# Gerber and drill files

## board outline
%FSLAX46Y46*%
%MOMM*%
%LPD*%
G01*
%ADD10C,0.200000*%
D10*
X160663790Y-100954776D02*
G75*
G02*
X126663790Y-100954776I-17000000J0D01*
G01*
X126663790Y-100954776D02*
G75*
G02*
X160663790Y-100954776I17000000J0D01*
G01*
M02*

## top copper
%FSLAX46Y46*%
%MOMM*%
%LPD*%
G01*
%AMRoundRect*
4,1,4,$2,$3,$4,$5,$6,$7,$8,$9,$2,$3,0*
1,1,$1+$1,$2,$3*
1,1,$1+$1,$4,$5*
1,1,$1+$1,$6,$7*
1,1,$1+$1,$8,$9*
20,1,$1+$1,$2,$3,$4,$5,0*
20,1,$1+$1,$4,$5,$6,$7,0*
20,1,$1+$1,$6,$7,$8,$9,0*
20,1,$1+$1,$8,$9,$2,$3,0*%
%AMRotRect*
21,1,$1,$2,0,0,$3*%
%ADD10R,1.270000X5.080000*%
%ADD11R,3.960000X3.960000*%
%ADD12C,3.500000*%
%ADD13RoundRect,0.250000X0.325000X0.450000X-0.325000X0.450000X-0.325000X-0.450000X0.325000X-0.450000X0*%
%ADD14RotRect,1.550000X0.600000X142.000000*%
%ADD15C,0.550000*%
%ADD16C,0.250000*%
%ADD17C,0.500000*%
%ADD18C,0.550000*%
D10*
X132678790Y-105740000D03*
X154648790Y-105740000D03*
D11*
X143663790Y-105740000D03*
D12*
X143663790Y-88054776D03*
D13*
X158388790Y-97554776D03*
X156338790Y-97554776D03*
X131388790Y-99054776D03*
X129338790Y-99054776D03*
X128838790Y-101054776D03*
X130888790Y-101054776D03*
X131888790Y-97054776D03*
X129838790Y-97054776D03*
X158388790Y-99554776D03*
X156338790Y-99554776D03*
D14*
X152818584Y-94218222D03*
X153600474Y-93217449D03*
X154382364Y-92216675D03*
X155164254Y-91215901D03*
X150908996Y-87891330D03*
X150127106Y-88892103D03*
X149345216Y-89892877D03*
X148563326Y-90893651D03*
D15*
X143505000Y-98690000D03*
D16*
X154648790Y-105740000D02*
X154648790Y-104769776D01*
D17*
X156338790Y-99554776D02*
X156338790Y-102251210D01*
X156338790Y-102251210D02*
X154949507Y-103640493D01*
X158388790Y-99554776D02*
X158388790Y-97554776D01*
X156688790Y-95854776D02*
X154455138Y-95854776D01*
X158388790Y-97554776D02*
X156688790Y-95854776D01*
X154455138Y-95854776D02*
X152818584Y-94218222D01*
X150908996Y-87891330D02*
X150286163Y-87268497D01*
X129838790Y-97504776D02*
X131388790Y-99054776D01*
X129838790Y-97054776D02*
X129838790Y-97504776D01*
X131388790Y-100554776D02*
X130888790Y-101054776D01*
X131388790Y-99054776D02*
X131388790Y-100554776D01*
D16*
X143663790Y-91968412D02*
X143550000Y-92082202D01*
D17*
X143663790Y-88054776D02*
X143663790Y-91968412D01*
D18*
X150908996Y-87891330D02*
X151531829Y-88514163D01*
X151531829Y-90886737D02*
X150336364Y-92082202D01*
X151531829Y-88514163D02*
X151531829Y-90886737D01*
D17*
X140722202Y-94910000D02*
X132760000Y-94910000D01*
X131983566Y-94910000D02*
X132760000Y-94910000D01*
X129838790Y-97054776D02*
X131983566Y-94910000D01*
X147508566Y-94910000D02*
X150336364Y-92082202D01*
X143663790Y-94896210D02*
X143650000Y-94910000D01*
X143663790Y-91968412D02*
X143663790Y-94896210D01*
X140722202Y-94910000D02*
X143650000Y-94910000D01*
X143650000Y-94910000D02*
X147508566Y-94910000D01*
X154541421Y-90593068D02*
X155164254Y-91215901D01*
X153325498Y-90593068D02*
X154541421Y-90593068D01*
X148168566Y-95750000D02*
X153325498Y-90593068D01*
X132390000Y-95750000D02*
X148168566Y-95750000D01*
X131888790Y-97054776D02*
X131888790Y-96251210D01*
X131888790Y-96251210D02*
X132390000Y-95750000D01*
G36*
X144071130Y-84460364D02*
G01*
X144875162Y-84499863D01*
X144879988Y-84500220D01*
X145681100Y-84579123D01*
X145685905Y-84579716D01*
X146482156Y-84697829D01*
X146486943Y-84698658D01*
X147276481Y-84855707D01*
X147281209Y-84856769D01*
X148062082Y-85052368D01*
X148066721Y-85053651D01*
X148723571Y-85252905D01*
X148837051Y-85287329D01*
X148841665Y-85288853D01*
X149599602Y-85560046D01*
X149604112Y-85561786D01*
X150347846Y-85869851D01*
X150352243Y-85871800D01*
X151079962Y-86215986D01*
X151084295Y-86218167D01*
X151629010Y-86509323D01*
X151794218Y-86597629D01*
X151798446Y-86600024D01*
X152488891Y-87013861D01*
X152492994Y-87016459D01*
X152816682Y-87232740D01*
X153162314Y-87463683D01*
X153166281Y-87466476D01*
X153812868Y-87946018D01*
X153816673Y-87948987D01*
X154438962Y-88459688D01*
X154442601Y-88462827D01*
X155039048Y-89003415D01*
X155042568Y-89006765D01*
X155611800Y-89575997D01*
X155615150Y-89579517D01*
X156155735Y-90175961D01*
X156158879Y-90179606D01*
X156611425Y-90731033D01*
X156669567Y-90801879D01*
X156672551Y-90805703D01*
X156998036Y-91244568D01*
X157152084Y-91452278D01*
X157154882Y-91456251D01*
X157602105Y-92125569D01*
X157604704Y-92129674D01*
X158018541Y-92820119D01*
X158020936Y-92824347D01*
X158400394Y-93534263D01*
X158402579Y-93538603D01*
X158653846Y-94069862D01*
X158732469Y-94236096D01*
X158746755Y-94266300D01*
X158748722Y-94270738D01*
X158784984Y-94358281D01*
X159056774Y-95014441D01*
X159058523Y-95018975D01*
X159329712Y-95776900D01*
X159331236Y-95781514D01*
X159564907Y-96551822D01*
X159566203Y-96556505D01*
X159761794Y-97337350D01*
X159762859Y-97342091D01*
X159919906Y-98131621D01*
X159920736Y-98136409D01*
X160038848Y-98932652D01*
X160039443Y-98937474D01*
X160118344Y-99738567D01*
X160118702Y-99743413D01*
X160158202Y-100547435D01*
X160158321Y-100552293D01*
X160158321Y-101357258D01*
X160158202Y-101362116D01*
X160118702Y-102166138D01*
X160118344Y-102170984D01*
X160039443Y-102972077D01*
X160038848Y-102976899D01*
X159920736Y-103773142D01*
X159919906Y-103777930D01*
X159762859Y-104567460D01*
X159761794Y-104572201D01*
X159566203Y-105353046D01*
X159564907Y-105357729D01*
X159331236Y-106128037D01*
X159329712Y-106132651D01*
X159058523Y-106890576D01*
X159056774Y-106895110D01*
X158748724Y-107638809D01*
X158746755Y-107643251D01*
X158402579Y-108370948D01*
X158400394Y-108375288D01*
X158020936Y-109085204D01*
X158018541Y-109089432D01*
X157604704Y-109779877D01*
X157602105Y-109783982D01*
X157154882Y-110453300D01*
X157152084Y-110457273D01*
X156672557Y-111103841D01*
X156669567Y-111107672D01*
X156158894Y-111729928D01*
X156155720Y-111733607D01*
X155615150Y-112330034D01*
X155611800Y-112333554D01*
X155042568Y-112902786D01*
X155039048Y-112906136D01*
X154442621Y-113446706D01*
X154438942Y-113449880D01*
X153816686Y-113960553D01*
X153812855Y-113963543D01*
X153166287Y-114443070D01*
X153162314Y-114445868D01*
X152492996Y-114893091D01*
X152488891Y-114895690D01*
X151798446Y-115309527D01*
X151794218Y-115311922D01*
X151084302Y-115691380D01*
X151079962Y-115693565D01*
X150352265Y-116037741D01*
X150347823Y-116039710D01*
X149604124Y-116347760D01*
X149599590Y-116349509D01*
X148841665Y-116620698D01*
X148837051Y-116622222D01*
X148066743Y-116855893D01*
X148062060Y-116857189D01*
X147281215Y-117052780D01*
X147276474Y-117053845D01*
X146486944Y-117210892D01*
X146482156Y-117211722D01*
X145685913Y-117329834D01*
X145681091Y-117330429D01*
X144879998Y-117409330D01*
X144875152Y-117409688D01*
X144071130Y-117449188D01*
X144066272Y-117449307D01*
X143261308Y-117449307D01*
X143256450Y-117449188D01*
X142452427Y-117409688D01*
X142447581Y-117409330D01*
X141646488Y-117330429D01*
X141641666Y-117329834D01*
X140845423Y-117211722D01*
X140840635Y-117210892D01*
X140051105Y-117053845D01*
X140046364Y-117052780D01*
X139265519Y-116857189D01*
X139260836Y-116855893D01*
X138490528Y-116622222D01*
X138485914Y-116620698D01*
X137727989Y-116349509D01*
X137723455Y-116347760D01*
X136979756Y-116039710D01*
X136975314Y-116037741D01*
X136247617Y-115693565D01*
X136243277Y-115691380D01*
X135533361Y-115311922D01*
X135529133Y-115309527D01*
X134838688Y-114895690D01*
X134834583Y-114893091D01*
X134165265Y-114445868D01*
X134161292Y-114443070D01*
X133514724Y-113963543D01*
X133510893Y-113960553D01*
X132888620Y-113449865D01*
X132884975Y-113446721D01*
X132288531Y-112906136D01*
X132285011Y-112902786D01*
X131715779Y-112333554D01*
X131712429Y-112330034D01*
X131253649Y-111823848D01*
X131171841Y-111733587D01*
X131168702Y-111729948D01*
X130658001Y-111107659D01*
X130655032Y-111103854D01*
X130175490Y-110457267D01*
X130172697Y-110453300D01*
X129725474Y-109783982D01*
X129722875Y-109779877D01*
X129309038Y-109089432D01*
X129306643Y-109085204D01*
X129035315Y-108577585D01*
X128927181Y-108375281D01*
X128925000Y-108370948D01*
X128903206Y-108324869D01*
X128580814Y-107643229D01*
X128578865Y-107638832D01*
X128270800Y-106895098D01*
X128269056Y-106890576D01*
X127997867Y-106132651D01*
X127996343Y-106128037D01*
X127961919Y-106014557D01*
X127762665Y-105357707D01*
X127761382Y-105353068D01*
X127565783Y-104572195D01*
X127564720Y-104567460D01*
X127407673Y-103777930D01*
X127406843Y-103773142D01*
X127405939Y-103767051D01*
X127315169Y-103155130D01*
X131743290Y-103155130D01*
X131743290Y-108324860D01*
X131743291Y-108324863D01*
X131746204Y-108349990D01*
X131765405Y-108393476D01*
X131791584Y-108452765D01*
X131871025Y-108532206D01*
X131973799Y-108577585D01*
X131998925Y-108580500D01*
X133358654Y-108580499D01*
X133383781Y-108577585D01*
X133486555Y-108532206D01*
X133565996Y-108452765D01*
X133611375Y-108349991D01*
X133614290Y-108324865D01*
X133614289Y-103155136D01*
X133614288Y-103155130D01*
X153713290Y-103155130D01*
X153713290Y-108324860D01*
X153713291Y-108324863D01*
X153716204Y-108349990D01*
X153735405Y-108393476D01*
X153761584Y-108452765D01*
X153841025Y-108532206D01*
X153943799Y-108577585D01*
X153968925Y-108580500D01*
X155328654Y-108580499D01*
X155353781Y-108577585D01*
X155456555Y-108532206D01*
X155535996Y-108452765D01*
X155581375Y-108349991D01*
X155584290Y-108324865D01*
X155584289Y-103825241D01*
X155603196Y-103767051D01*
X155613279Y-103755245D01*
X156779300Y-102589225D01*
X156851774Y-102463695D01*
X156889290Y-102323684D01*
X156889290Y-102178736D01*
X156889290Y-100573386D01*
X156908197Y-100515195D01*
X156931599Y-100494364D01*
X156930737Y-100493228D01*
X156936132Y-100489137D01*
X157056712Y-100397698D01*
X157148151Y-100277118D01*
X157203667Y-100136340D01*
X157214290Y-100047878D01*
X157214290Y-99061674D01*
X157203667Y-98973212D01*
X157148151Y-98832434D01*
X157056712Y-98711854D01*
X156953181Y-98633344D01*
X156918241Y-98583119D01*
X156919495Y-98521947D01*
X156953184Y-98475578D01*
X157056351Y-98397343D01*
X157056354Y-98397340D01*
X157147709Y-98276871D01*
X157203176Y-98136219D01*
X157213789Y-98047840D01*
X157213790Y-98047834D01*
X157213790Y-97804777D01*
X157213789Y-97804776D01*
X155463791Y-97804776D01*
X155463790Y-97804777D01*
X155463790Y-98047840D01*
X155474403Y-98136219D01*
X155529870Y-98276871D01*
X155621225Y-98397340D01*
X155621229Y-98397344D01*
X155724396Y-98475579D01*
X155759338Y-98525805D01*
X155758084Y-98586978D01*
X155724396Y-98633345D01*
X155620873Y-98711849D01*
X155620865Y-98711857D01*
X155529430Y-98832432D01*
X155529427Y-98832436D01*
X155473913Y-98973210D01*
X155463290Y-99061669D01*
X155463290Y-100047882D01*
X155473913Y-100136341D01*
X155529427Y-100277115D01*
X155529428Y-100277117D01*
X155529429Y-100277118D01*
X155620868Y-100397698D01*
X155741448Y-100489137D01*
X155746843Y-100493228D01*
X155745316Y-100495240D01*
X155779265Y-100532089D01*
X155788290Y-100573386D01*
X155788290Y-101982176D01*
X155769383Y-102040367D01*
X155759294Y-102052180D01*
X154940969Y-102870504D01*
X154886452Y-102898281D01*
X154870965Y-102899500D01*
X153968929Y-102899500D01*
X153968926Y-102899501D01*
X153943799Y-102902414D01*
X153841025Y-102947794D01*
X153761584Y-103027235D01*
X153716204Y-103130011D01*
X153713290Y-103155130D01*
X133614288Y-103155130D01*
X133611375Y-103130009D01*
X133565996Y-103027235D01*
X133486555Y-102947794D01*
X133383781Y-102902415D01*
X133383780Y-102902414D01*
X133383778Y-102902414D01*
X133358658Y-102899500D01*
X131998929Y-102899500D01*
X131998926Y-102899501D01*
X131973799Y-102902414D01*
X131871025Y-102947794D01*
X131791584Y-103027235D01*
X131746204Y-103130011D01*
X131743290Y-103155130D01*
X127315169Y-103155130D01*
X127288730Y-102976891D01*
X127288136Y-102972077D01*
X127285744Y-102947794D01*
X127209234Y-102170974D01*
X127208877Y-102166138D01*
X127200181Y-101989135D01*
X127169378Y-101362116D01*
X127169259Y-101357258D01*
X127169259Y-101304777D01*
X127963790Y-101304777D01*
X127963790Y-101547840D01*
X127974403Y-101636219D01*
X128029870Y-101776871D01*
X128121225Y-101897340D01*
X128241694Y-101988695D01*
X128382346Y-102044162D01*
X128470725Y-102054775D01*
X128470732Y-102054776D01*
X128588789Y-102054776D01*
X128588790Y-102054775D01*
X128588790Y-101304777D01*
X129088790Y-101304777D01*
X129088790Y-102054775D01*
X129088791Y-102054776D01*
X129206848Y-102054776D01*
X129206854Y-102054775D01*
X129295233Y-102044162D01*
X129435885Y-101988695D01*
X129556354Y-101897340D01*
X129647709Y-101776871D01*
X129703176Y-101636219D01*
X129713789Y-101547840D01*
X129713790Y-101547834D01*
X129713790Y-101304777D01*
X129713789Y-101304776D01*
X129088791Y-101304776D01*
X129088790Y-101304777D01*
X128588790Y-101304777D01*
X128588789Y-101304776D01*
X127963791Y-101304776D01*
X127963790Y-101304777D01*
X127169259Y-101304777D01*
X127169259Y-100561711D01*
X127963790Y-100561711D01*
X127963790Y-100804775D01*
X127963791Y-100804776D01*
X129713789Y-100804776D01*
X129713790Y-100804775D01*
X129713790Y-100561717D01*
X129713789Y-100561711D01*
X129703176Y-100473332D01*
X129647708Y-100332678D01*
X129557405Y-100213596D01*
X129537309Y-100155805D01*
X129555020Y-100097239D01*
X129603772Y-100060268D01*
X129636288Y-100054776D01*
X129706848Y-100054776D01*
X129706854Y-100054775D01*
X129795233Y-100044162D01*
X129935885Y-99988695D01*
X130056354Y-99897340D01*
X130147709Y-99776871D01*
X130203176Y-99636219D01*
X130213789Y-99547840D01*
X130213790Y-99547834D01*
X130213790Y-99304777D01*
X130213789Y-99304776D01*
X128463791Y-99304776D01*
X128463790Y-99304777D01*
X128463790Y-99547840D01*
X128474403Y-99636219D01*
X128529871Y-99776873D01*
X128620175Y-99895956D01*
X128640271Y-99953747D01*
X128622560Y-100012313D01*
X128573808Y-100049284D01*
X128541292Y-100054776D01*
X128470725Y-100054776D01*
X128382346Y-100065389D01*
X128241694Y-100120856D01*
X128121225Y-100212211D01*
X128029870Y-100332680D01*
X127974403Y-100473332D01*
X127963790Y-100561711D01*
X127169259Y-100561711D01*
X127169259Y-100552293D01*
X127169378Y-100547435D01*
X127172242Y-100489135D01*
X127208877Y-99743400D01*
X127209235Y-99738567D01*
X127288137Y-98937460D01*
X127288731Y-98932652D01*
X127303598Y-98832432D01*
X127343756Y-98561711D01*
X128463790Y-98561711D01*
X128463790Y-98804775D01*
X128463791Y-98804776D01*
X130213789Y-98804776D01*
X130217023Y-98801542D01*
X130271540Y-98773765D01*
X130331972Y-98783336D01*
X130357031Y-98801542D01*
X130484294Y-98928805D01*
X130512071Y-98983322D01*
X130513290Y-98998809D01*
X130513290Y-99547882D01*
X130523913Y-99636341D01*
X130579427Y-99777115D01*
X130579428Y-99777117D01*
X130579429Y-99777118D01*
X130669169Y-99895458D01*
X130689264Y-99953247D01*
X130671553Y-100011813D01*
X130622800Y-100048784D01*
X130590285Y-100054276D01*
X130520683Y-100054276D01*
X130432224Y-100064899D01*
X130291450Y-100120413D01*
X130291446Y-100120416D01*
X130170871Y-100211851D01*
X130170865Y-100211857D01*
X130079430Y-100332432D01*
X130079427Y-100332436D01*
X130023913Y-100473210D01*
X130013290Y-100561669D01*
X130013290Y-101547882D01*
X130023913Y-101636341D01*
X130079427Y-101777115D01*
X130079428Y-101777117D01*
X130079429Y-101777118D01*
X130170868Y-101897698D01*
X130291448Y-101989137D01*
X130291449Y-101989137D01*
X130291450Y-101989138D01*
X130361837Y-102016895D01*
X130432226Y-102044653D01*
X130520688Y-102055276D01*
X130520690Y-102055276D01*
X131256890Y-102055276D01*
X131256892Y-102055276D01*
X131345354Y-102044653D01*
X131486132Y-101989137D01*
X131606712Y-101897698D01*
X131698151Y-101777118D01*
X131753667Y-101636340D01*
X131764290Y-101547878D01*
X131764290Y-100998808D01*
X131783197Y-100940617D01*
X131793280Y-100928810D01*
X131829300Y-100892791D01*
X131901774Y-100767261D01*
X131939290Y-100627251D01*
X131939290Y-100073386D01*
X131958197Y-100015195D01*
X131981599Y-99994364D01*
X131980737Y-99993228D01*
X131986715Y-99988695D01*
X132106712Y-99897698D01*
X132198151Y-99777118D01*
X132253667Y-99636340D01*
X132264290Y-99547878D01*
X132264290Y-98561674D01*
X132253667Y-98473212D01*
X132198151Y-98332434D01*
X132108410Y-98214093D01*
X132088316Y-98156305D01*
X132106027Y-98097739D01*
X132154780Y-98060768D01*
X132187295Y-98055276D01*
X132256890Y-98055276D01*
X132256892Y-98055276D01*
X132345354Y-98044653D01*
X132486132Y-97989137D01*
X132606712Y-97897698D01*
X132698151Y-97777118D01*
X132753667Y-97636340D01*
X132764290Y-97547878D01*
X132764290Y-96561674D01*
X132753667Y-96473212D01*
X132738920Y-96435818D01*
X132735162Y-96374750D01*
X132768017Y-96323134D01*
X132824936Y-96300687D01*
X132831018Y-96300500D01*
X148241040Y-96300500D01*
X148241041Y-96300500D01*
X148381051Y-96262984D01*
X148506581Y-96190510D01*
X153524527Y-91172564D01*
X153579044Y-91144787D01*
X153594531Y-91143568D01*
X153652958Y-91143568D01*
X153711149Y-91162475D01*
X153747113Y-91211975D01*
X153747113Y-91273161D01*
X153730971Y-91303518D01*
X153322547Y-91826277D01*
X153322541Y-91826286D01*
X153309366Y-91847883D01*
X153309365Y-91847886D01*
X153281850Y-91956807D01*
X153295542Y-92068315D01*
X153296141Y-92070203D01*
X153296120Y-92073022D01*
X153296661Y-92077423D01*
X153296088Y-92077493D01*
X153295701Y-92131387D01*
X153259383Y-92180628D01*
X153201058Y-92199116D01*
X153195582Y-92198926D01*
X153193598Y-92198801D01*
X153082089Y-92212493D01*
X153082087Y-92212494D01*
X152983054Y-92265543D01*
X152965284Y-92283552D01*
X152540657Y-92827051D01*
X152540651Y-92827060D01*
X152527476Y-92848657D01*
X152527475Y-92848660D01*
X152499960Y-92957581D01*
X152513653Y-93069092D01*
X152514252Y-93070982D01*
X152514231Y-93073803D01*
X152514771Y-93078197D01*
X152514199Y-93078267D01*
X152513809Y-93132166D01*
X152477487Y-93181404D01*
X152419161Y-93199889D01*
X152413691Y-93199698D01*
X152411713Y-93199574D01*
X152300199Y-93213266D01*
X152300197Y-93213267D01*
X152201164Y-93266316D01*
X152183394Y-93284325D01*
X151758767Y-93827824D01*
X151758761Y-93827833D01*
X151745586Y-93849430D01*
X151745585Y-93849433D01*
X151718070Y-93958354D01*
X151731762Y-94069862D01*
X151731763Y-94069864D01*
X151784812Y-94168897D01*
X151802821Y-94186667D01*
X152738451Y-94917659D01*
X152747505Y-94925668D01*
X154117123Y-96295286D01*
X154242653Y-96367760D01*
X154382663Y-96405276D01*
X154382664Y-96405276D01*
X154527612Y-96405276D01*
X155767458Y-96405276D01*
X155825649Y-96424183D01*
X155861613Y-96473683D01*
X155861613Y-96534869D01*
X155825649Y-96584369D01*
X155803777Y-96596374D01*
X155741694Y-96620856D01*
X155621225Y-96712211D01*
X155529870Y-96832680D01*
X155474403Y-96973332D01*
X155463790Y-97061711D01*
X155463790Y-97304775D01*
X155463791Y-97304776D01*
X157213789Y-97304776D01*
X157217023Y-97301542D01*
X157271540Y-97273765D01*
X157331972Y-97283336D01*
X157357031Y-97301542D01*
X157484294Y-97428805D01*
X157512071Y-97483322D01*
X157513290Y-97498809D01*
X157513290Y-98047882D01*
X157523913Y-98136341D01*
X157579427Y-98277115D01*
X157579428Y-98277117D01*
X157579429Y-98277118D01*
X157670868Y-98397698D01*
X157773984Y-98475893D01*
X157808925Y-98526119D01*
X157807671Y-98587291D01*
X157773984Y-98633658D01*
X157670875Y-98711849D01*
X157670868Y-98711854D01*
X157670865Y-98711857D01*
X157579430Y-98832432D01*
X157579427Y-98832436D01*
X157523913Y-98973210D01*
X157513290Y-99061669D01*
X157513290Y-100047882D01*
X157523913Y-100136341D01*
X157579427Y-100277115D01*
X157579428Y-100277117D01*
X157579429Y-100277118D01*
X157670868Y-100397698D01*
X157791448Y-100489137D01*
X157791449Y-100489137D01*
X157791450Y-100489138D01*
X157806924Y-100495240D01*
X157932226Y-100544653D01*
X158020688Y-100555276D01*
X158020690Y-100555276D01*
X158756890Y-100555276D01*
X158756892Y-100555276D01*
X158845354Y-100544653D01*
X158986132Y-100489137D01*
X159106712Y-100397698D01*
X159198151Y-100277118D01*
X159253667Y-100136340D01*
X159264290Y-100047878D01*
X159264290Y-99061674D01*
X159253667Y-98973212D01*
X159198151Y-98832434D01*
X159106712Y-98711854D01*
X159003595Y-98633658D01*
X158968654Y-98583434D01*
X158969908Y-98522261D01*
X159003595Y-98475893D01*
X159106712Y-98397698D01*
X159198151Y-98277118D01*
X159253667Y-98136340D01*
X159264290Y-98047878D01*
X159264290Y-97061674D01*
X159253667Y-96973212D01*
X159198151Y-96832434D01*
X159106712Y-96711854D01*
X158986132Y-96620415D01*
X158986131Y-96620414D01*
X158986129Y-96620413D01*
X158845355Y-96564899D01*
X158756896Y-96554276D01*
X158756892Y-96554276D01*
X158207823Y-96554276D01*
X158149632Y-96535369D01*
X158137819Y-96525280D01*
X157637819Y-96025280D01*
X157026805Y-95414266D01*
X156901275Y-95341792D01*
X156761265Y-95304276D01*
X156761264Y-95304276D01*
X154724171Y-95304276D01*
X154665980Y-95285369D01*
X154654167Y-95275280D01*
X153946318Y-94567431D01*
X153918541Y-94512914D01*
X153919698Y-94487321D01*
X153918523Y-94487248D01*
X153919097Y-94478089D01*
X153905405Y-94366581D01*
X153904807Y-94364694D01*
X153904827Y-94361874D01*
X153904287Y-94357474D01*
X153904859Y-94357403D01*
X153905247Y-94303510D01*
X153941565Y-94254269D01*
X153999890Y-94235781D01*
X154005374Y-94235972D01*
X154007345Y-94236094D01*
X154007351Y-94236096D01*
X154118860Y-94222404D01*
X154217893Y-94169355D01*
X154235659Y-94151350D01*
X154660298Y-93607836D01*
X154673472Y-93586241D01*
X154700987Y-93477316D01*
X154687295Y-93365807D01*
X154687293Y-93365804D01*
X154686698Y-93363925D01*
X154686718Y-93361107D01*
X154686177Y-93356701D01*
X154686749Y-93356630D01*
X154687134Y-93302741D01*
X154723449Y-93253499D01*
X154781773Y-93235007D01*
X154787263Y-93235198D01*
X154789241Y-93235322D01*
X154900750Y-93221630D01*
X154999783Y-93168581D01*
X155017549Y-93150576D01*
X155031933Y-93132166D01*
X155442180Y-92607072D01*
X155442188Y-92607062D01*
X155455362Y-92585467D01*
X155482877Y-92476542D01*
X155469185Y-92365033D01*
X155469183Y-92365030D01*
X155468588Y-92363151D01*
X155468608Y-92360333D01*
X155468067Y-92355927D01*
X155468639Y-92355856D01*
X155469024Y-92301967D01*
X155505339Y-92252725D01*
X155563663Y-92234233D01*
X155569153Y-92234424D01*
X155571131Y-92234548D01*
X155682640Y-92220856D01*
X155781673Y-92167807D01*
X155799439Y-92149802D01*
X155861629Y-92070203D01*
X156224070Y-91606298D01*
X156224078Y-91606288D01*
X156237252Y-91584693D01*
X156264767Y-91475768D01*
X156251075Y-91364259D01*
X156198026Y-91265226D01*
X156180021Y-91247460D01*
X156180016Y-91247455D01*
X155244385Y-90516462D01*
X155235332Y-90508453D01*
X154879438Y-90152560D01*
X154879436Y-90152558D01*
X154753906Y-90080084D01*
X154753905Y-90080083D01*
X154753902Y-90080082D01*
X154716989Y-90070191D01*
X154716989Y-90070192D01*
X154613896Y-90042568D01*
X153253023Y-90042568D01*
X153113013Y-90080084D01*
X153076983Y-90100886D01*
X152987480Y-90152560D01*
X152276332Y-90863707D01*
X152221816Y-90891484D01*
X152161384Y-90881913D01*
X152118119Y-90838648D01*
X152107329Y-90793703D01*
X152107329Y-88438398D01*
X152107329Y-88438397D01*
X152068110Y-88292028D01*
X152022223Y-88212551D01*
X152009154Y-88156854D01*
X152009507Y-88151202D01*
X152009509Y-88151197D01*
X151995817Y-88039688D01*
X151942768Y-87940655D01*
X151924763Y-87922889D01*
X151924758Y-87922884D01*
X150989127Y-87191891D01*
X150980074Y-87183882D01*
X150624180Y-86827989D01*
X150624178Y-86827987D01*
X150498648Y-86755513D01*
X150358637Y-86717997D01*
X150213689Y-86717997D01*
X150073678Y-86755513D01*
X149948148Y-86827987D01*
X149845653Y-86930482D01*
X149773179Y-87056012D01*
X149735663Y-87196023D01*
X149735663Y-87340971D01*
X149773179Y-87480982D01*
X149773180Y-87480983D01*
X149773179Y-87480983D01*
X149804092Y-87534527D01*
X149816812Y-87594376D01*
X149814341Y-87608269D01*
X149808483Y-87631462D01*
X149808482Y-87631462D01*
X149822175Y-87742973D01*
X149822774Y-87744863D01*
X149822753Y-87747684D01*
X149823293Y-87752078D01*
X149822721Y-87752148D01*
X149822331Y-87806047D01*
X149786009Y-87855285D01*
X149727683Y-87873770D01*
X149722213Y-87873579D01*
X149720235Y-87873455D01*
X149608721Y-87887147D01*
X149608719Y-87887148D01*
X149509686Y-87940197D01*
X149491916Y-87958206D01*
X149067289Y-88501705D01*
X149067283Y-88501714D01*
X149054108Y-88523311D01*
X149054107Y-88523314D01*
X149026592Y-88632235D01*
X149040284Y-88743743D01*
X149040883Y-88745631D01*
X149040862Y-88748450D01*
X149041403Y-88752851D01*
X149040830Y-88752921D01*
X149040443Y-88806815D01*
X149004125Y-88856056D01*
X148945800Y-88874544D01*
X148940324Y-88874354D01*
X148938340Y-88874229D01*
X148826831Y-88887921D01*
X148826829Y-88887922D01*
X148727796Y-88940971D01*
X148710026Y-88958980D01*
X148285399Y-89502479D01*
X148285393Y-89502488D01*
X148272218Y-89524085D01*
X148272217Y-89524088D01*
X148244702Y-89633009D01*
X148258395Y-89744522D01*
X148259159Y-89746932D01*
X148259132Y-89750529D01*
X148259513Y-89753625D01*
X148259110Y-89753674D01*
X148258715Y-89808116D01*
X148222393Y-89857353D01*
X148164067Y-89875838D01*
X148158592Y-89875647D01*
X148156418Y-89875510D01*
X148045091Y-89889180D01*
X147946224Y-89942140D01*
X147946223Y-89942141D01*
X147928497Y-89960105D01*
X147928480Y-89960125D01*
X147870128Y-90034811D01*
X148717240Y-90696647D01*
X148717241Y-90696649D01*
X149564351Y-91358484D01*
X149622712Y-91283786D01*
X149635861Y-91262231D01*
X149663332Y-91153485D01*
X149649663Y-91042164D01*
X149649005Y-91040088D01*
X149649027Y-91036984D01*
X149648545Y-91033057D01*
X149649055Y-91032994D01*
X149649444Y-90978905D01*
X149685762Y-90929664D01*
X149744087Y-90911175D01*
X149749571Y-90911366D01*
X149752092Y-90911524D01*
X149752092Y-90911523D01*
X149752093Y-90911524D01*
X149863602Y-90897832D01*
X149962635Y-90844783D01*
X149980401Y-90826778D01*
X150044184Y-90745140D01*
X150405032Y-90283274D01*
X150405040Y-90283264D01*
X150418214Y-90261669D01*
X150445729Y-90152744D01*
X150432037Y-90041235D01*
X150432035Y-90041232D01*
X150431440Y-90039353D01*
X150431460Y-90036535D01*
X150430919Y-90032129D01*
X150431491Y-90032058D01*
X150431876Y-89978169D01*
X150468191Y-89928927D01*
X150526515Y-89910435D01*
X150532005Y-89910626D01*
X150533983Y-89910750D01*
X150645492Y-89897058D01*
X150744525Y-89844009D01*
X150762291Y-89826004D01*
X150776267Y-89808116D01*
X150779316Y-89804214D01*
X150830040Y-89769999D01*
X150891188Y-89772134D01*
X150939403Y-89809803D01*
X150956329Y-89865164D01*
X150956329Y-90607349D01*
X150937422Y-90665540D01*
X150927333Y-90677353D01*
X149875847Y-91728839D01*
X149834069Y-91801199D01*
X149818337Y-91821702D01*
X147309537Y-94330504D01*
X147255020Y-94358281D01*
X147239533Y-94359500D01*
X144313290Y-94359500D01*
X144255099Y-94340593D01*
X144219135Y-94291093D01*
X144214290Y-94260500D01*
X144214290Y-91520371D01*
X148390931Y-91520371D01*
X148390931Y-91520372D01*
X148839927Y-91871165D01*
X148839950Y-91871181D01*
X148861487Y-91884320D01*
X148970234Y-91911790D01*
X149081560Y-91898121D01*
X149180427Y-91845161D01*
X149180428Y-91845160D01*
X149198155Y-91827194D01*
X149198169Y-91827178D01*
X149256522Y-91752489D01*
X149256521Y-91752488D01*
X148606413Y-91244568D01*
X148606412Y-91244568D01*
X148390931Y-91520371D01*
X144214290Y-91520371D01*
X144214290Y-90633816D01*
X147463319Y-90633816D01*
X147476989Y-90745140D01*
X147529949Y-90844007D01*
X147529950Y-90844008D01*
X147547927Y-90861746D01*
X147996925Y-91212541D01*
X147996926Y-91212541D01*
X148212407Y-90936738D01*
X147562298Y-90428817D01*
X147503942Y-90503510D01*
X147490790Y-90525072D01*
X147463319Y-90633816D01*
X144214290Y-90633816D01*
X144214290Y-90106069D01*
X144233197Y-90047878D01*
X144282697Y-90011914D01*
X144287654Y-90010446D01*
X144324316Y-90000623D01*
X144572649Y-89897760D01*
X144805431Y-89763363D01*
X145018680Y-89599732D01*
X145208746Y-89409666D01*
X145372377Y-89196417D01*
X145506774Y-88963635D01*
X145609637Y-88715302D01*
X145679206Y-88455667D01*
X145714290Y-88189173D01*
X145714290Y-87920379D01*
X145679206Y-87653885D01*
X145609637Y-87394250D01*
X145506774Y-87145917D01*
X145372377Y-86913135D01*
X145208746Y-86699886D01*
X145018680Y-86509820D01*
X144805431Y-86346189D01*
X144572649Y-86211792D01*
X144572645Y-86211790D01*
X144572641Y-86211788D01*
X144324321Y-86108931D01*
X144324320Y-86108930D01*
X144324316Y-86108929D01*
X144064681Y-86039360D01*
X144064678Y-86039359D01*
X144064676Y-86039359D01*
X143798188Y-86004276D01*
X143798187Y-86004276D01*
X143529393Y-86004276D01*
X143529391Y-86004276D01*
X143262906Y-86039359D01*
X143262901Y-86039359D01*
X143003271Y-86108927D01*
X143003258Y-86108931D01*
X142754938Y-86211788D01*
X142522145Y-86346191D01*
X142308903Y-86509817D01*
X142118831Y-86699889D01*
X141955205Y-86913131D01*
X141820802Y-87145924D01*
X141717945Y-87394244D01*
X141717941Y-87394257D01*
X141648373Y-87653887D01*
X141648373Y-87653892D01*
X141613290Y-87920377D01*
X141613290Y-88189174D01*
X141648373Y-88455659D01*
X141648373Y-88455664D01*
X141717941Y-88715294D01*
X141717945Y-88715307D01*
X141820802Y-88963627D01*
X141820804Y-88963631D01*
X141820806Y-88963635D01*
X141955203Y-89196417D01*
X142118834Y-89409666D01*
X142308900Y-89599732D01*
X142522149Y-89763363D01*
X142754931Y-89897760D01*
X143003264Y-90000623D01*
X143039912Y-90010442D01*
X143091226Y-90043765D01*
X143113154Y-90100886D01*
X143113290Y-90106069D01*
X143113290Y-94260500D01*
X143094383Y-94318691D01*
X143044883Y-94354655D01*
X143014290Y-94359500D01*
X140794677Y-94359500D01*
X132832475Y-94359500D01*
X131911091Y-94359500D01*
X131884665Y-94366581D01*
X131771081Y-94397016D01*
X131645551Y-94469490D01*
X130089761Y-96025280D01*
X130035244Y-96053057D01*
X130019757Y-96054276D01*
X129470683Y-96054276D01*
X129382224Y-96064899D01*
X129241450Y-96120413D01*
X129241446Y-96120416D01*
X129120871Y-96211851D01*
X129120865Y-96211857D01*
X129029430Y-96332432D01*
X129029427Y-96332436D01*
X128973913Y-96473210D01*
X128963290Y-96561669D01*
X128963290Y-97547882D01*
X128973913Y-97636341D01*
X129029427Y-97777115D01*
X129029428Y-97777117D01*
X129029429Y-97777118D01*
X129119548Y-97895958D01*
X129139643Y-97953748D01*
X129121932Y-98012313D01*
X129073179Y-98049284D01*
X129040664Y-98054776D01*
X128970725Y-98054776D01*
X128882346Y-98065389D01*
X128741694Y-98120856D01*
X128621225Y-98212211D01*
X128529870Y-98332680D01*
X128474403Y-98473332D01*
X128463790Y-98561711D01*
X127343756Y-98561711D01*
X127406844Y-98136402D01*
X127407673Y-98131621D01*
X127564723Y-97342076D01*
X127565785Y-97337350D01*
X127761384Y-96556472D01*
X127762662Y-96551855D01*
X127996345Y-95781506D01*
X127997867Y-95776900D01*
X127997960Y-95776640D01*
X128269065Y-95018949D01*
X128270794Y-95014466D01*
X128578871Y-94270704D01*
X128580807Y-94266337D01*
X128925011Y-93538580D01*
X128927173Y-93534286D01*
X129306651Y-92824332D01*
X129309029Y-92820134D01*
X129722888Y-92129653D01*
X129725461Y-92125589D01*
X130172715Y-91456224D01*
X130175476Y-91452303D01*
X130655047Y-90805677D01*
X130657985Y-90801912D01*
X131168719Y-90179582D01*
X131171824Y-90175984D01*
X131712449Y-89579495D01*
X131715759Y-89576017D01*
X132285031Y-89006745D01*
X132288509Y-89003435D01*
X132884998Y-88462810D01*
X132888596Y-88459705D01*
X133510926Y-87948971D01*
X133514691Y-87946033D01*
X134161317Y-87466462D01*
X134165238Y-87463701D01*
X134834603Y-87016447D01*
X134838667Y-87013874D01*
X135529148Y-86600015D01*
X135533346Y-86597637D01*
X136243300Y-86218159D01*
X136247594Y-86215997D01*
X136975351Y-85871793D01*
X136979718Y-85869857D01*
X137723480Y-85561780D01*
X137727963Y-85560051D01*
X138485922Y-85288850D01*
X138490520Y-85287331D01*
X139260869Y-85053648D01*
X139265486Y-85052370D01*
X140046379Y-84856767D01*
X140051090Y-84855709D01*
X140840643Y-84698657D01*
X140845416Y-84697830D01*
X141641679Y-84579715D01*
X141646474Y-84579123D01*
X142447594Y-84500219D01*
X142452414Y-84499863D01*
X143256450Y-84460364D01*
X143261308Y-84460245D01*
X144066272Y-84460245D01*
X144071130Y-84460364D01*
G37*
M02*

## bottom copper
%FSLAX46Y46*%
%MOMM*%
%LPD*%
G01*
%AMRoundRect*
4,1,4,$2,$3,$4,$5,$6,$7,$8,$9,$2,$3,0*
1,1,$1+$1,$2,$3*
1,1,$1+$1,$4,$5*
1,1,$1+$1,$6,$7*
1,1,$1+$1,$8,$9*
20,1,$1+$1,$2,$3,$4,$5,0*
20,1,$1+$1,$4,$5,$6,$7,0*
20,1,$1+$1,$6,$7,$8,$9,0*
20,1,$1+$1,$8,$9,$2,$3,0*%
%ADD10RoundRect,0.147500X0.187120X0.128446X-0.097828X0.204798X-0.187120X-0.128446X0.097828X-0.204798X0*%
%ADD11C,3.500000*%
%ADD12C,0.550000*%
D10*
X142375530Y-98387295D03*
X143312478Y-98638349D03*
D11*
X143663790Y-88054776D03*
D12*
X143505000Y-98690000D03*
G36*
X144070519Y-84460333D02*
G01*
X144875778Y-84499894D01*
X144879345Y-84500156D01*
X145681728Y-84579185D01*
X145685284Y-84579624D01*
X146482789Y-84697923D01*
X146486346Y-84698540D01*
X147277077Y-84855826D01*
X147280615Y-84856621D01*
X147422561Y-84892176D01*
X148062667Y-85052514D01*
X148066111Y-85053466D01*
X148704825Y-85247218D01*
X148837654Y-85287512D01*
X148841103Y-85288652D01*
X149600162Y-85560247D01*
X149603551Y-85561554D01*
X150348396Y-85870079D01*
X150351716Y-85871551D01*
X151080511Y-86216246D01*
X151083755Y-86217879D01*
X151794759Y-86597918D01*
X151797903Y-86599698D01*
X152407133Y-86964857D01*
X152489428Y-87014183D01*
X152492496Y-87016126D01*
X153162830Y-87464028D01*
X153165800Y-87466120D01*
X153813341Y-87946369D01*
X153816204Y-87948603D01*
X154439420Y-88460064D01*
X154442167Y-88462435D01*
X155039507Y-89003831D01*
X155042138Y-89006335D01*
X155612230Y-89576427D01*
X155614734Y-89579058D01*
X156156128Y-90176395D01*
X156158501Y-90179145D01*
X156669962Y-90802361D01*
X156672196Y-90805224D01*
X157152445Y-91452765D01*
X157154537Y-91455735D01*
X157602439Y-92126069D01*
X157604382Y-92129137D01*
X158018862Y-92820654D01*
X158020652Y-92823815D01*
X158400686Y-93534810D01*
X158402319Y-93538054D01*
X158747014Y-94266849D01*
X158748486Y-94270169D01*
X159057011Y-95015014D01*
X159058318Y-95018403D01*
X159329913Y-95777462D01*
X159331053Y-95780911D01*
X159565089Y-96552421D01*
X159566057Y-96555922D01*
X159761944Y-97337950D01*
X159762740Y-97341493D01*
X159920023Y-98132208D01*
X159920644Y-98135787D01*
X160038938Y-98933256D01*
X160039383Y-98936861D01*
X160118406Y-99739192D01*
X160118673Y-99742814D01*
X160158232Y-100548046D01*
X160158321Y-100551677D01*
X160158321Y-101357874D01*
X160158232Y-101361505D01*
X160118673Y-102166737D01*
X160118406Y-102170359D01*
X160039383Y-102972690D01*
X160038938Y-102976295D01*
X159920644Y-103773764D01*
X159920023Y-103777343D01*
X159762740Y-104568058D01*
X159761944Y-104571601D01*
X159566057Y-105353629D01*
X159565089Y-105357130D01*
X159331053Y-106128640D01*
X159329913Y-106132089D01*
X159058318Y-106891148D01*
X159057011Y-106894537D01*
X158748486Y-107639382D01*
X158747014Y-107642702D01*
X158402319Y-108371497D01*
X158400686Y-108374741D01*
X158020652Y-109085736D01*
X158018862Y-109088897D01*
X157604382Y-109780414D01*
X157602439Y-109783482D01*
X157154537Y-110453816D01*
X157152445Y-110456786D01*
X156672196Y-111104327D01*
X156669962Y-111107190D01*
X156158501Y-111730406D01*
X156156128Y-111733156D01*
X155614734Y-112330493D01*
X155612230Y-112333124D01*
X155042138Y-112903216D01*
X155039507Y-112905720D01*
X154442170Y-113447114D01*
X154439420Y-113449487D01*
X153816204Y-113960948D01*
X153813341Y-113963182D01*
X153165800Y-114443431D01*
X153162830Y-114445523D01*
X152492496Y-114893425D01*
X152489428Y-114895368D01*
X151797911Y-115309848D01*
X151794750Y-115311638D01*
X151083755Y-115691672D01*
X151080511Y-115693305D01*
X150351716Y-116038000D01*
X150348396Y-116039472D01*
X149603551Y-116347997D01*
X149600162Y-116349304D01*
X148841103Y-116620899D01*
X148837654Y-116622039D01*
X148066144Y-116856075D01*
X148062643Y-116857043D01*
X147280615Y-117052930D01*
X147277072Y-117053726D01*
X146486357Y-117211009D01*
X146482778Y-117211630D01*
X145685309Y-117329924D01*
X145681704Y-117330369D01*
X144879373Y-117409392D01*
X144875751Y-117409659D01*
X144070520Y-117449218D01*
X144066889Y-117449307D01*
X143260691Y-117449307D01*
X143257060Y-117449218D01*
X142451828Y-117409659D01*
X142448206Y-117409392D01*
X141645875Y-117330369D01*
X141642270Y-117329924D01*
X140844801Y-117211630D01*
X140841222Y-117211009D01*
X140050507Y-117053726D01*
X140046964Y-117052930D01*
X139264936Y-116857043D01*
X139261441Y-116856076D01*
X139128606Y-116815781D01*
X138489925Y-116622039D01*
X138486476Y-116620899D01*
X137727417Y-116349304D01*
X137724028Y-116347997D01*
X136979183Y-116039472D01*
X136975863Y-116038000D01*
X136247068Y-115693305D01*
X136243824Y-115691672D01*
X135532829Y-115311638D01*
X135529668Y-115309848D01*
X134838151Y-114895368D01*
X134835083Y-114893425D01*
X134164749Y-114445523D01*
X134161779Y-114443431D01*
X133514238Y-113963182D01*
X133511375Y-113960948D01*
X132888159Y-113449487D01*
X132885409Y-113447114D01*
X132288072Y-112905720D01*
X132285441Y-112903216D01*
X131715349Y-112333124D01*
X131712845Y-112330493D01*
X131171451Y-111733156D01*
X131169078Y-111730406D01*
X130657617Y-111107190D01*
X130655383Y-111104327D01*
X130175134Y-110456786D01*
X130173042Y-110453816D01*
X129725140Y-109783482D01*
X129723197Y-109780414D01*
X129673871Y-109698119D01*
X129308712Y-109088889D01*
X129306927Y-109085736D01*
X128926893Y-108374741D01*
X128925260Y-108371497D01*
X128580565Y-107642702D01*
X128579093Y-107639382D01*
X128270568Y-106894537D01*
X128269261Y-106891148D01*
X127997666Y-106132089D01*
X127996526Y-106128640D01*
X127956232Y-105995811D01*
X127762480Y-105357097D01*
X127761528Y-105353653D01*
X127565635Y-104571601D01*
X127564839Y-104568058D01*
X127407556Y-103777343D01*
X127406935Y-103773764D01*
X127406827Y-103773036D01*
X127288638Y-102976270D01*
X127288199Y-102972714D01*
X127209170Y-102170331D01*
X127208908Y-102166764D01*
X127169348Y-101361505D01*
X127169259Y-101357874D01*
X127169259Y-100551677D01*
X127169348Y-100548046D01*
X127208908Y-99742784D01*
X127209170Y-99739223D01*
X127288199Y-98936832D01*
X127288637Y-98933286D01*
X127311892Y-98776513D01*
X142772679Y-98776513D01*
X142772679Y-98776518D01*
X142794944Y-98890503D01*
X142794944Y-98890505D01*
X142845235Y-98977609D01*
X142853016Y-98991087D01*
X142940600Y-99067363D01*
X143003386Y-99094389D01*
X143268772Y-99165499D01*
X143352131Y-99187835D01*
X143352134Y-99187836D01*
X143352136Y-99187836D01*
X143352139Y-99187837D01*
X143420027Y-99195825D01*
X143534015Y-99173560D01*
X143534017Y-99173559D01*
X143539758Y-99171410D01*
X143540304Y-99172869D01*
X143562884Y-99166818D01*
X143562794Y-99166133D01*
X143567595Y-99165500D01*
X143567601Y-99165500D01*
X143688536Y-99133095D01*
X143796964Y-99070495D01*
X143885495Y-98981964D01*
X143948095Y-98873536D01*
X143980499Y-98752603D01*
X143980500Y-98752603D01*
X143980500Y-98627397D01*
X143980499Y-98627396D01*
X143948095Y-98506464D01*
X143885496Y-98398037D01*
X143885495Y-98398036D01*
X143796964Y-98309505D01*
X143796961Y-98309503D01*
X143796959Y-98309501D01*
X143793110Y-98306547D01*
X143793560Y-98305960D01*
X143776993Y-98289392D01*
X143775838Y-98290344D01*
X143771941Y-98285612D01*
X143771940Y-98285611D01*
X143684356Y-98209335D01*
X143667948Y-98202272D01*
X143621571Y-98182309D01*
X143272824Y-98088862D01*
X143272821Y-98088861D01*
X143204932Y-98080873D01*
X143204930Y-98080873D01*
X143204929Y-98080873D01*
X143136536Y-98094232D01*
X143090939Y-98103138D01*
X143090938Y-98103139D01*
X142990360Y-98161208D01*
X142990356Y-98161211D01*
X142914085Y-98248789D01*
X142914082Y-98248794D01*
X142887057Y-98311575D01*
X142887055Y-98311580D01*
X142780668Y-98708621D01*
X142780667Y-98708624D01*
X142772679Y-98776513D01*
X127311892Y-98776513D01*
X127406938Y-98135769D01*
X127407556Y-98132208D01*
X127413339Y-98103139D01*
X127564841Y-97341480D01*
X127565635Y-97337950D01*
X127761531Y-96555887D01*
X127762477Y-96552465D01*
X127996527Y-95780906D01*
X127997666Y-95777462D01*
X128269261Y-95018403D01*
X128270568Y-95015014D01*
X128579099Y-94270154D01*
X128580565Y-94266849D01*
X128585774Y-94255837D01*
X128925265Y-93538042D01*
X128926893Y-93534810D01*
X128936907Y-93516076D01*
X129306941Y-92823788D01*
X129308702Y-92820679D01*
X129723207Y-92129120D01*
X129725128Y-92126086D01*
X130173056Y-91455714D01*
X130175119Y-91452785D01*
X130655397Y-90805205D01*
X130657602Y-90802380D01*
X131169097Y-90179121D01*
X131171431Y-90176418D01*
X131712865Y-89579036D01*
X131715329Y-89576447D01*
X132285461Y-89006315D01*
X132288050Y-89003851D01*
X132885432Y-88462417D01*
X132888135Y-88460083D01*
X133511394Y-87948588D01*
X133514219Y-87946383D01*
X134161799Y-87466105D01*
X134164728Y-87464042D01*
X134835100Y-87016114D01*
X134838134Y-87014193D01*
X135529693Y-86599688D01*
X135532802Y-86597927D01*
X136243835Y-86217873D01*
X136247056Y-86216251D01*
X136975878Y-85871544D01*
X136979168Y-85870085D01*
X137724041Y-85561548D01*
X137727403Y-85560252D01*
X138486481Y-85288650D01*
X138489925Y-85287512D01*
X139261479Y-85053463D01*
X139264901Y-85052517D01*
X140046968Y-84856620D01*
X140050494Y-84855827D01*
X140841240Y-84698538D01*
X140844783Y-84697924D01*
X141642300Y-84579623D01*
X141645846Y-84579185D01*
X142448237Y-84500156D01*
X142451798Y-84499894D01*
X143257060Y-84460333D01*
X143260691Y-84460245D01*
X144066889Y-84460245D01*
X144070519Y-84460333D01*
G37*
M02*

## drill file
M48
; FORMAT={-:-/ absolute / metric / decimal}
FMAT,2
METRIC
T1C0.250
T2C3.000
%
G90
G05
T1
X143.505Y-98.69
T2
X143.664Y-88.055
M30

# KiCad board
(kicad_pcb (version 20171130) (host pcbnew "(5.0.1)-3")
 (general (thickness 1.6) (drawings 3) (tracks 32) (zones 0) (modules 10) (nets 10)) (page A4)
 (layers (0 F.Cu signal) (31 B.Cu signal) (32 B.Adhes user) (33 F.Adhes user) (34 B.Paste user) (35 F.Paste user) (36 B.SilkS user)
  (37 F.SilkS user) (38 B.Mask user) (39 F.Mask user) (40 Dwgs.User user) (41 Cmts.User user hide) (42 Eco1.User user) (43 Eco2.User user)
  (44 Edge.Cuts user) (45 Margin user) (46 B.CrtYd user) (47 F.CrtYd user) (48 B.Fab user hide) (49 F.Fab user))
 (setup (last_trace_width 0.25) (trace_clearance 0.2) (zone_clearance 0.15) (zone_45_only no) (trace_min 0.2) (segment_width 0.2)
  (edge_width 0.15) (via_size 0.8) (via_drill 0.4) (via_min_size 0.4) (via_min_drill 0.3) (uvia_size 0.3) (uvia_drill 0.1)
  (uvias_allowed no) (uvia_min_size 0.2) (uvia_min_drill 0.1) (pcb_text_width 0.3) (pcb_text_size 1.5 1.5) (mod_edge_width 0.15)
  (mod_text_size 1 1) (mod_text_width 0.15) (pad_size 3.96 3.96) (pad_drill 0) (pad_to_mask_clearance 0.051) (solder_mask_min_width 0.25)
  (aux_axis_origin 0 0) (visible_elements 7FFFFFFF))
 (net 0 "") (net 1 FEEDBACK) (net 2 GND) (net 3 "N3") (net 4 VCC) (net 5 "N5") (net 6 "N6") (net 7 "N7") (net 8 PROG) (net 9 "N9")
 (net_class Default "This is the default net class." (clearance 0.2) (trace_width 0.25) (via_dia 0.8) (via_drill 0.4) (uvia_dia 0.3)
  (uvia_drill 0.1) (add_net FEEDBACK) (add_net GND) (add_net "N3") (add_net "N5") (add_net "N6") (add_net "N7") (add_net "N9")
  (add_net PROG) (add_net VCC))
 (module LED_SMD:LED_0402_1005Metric (layer B.Cu) (at 142.844004 98.512822 165)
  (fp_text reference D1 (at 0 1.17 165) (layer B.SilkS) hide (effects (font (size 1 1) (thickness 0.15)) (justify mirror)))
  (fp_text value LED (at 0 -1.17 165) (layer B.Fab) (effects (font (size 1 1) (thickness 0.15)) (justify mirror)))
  (pad 2 smd roundrect (at 0.485 0 165) (size 0.59 0.64) (layers B.Cu B.Paste B.Mask) (roundrect_rratio 0.25) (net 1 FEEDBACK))
  (pad 1 smd roundrect (at -0.485 0 165) (size 0.59 0.64) (layers B.Cu B.Paste B.Mask) (roundrect_rratio 0.25) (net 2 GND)))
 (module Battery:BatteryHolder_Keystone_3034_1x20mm (layer F.Cu) (at 143.66379 105.74)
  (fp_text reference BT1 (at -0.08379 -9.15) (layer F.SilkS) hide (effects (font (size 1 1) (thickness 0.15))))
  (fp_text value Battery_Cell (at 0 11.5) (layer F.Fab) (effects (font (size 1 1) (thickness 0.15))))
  (pad 1 smd rect (at -10.985 0) (size 1.27 5.08) (layers F.Cu F.Paste F.Mask) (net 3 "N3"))
  (pad 1 smd rect (at 10.985 0) (size 1.27 5.08) (layers F.Cu F.Paste F.Mask) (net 3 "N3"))
  (pad 2 smd rect (at 0 0) (size 3.96 3.96) (layers F.Cu F.Paste F.Mask) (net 2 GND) (zone_connect 2)))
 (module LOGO (layer B.Cu) (at 144.12 102.37 180)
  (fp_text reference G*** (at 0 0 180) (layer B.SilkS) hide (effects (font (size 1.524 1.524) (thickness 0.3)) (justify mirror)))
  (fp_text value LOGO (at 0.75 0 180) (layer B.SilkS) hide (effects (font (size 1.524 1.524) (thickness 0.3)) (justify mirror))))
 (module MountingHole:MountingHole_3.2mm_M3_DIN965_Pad (layer B.Cu) (at 143.66379 88.054776 180)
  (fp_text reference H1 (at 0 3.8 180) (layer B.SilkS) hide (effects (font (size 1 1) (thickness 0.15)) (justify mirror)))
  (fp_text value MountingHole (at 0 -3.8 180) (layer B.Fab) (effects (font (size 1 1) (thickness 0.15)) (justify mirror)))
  (pad 1 thru_hole circle (at 0 0 180) (size 3.5 3.5) (drill 3) (layers *.Cu *.Mask) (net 1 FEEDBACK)))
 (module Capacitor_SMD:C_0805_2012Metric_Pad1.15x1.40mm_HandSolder (layer F.Cu) (at 157.36379 97.554776 180)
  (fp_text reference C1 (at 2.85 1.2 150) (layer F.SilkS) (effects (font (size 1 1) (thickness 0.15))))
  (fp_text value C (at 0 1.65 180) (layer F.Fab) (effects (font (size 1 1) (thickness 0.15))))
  (pad 1 smd roundrect (at -1.025 0 180) (size 1.15 1.4) (layers F.Cu F.Paste F.Mask) (roundrect_rratio 0.217391) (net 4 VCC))
  (pad 2 smd roundrect (at 1.025 0 180) (size 1.15 1.4) (layers F.Cu F.Paste F.Mask) (roundrect_rratio 0.217391) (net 2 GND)))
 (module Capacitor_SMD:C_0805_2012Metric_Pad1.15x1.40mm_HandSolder (layer F.Cu) (at 130.36379 99.054776 180)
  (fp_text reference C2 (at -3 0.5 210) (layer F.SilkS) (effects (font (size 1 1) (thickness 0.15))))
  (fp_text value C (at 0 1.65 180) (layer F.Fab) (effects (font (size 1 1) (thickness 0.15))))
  (pad 1 smd roundrect (at -1.025 0 180) (size 1.15 1.4) (layers F.Cu F.Paste F.Mask) (roundrect_rratio 0.217391) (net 1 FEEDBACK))
  (pad 2 smd roundrect (at 1.025 0 180) (size 1.15 1.4) (layers F.Cu F.Paste F.Mask) (roundrect_rratio 0.217391) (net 2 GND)))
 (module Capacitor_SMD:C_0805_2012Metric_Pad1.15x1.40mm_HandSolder (layer F.Cu) (at 129.86379 101.054776 180)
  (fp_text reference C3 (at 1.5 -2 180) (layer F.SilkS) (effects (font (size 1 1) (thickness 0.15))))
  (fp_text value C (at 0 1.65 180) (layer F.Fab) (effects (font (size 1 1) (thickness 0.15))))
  (pad 2 smd roundrect (at 1.025 0 180) (size 1.15 1.4) (layers F.Cu F.Paste F.Mask) (roundrect_rratio 0.217391) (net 2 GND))
  (pad 1 smd roundrect (at -1.025 0 180) (size 1.15 1.4) (layers F.Cu F.Paste F.Mask) (roundrect_rratio 0.217391) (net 1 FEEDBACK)))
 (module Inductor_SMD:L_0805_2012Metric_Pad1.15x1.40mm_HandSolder (layer F.Cu) (at 130.86379 97.054776 180)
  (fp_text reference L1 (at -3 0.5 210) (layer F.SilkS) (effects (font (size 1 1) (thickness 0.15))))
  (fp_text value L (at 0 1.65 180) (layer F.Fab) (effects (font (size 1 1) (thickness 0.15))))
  (pad 1 smd roundrect (at -1.025 0 180) (size 1.15 1.4) (layers F.Cu F.Paste F.Mask) (roundrect_rratio 0.217391) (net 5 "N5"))
  (pad 2 smd roundrect (at 1.025 0 180) (size 1.15 1.4) (layers F.Cu F.Paste F.Mask) (roundrect_rratio 0.217391) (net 1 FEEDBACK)))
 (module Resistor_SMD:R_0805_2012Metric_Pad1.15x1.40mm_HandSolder (layer F.Cu) (at 157.36379 99.554776 180)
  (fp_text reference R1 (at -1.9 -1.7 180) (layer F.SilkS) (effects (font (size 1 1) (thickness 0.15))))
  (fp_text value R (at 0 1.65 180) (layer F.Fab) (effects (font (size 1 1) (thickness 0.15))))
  (pad 1 smd roundrect (at -1.025 0 180) (size 1.15 1.4) (layers F.Cu F.Paste F.Mask) (roundrect_rratio 0.217391) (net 4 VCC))
  (pad 2 smd roundrect (at 1.025 0 180) (size 1.15 1.4) (layers F.Cu F.Paste F.Mask) (roundrect_rratio 0.217391) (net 3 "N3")))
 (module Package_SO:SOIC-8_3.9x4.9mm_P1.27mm (layer F.Cu) (at 151.86379 91.054776 142)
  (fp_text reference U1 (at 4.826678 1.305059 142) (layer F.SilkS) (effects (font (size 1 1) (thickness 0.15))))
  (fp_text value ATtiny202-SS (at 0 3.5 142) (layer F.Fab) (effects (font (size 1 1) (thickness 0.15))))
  (pad 1 smd rect (at -2.7 -1.905 142) (size 1.55 0.6) (layers F.Cu F.Paste F.Mask) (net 4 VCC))
  (pad 2 smd rect (at -2.7 -0.635 142) (size 1.55 0.6) (layers F.Cu F.Paste F.Mask) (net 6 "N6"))
  (pad 3 smd rect (at -2.7 0.635 142) (size 1.55 0.6) (layers F.Cu F.Paste F.Mask) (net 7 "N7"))
  (pad 4 smd rect (at -2.7 1.905 142) (size 1.55 0.6) (layers F.Cu F.Paste F.Mask) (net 5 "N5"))
  (pad 5 smd rect (at 2.7 1.905 142) (size 1.55 0.6) (layers F.Cu F.Paste F.Mask) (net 1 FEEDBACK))
  (pad 6 smd rect (at 2.7 0.635 142) (size 1.55 0.6) (layers F.Cu F.Paste F.Mask) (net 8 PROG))
  (pad 7 smd rect (at 2.7 -0.635 142) (size 1.55 0.6) (layers F.Cu F.Paste F.Mask) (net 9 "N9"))
  (pad 8 smd rect (at 2.7 -1.905 142) (size 1.55 0.6) (layers F.Cu F.Paste F.Mask) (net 2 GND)))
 (gr_circle (center 143.66379 100.954776) (end 126.66379 100.954776) (layer Edge.Cuts) (width 0.2))
 (via (at 143.505 98.69) (size 0.55) (drill 0.25) (layers F.Cu B.Cu) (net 2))
 (segment (start 154.64879 105.74) (end 154.64879 104.769776) (width 0.25) (layer F.Cu) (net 3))
 (segment (start 156.33879 99.554776) (end 156.33879 102.25121) (width 0.5) (layer F.Cu) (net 3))
 (segment (start 156.33879 102.25121) (end 154.949507 103.640493) (width 0.5) (layer F.Cu) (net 3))
 (segment (start 158.38879 99.554776) (end 158.38879 97.554776) (width 0.5) (layer F.Cu) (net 4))
 (segment (start 156.68879 95.854776) (end 154.455138 95.854776) (width 0.5) (layer F.Cu) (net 4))
 (segment (start 158.38879 97.554776) (end 156.68879 95.854776) (width 0.5) (layer F.Cu) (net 4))
 (segment (start 154.455138 95.854776) (end 152.818584 94.218222) (width 0.5) (layer F.Cu) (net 4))
 (segment (start 150.908996 87.89133) (end 150.286163 87.268497) (width 0.5) (layer F.Cu) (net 1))
 (segment (start 129.83879 97.504776) (end 131.38879 99.054776) (width 0.5) (layer F.Cu) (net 1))
 (segment (start 129.83879 97.054776) (end 129.83879 97.504776) (width 0.5) (layer F.Cu) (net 1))
 (segment (start 131.38879 100.554776) (end 130.88879 101.054776) (width 0.5) (layer F.Cu) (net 1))
 (segment (start 131.38879 99.054776) (end 131.38879 100.554776) (width 0.5) (layer F.Cu) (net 1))
 (segment (start 143.66379 91.968412) (end 143.55 92.082202) (width 0.25) (layer F.Cu) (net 1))
 (segment (start 143.66379 88.054776) (end 143.66379 91.968412) (width 0.5) (layer F.Cu) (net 1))
 (segment (start 150.908996 87.89133) (end 151.531829 88.514163) (width 0.55) (layer F.Cu) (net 1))
 (segment (start 151.531829 90.886737) (end 150.336364 92.082202) (width 0.55) (layer F.Cu) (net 1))
 (segment (start 151.531829 88.514163) (end 151.531829 90.886737) (width 0.55) (layer F.Cu) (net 1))
 (segment (start 140.722202 94.91) (end 132.76 94.91) (width 0.5) (layer F.Cu) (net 1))
 (segment (start 131.983566 94.91) (end 132.76 94.91) (width 0.5) (layer F.Cu) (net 1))
 (segment (start 129.83879 97.054776) (end 131.983566 94.91) (width 0.5) (layer F.Cu) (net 1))
 (segment (start 147.508566 94.91) (end 150.336364 92.082202) (width 0.5) (layer F.Cu) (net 1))
 (segment (start 143.66379 94.89621) (end 143.65 94.91) (width 0.5) (layer F.Cu) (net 1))
 (segment (start 143.66379 91.968412) (end 143.66379 94.89621) (width 0.5) (layer F.Cu) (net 1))
 (segment (start 140.722202 94.91) (end 143.65 94.91) (width 0.5) (layer F.Cu) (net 1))
 (segment (start 143.65 94.91) (end 147.508566 94.91) (width 0.5) (layer F.Cu) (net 1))
 (segment (start 154.541421 90.593068) (end 155.164254 91.215901) (width 0.5) (layer F.Cu) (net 5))
 (segment (start 153.325498 90.593068) (end 154.541421 90.593068) (width 0.5) (layer F.Cu) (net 5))
 (segment (start 148.168566 95.75) (end 153.325498 90.593068) (width 0.5) (layer F.Cu) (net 5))
 (segment (start 132.39 95.75) (end 148.168566 95.75) (width 0.5) (layer F.Cu) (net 5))
 (segment (start 131.88879 97.054776) (end 131.88879 96.25121) (width 0.5) (layer F.Cu) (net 5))
 (segment (start 131.88879 96.25121) (end 132.39 95.75) (width 0.5) (layer F.Cu) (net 5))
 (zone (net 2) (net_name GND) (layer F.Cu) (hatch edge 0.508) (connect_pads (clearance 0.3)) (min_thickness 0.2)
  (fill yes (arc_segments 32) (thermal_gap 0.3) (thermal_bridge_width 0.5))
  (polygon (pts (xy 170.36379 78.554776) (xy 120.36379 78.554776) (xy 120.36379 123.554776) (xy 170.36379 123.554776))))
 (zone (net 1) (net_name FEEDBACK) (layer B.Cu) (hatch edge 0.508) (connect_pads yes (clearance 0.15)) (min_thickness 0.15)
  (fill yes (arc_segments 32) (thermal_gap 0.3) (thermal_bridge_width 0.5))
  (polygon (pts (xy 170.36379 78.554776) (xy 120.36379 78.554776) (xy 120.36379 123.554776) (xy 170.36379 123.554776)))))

